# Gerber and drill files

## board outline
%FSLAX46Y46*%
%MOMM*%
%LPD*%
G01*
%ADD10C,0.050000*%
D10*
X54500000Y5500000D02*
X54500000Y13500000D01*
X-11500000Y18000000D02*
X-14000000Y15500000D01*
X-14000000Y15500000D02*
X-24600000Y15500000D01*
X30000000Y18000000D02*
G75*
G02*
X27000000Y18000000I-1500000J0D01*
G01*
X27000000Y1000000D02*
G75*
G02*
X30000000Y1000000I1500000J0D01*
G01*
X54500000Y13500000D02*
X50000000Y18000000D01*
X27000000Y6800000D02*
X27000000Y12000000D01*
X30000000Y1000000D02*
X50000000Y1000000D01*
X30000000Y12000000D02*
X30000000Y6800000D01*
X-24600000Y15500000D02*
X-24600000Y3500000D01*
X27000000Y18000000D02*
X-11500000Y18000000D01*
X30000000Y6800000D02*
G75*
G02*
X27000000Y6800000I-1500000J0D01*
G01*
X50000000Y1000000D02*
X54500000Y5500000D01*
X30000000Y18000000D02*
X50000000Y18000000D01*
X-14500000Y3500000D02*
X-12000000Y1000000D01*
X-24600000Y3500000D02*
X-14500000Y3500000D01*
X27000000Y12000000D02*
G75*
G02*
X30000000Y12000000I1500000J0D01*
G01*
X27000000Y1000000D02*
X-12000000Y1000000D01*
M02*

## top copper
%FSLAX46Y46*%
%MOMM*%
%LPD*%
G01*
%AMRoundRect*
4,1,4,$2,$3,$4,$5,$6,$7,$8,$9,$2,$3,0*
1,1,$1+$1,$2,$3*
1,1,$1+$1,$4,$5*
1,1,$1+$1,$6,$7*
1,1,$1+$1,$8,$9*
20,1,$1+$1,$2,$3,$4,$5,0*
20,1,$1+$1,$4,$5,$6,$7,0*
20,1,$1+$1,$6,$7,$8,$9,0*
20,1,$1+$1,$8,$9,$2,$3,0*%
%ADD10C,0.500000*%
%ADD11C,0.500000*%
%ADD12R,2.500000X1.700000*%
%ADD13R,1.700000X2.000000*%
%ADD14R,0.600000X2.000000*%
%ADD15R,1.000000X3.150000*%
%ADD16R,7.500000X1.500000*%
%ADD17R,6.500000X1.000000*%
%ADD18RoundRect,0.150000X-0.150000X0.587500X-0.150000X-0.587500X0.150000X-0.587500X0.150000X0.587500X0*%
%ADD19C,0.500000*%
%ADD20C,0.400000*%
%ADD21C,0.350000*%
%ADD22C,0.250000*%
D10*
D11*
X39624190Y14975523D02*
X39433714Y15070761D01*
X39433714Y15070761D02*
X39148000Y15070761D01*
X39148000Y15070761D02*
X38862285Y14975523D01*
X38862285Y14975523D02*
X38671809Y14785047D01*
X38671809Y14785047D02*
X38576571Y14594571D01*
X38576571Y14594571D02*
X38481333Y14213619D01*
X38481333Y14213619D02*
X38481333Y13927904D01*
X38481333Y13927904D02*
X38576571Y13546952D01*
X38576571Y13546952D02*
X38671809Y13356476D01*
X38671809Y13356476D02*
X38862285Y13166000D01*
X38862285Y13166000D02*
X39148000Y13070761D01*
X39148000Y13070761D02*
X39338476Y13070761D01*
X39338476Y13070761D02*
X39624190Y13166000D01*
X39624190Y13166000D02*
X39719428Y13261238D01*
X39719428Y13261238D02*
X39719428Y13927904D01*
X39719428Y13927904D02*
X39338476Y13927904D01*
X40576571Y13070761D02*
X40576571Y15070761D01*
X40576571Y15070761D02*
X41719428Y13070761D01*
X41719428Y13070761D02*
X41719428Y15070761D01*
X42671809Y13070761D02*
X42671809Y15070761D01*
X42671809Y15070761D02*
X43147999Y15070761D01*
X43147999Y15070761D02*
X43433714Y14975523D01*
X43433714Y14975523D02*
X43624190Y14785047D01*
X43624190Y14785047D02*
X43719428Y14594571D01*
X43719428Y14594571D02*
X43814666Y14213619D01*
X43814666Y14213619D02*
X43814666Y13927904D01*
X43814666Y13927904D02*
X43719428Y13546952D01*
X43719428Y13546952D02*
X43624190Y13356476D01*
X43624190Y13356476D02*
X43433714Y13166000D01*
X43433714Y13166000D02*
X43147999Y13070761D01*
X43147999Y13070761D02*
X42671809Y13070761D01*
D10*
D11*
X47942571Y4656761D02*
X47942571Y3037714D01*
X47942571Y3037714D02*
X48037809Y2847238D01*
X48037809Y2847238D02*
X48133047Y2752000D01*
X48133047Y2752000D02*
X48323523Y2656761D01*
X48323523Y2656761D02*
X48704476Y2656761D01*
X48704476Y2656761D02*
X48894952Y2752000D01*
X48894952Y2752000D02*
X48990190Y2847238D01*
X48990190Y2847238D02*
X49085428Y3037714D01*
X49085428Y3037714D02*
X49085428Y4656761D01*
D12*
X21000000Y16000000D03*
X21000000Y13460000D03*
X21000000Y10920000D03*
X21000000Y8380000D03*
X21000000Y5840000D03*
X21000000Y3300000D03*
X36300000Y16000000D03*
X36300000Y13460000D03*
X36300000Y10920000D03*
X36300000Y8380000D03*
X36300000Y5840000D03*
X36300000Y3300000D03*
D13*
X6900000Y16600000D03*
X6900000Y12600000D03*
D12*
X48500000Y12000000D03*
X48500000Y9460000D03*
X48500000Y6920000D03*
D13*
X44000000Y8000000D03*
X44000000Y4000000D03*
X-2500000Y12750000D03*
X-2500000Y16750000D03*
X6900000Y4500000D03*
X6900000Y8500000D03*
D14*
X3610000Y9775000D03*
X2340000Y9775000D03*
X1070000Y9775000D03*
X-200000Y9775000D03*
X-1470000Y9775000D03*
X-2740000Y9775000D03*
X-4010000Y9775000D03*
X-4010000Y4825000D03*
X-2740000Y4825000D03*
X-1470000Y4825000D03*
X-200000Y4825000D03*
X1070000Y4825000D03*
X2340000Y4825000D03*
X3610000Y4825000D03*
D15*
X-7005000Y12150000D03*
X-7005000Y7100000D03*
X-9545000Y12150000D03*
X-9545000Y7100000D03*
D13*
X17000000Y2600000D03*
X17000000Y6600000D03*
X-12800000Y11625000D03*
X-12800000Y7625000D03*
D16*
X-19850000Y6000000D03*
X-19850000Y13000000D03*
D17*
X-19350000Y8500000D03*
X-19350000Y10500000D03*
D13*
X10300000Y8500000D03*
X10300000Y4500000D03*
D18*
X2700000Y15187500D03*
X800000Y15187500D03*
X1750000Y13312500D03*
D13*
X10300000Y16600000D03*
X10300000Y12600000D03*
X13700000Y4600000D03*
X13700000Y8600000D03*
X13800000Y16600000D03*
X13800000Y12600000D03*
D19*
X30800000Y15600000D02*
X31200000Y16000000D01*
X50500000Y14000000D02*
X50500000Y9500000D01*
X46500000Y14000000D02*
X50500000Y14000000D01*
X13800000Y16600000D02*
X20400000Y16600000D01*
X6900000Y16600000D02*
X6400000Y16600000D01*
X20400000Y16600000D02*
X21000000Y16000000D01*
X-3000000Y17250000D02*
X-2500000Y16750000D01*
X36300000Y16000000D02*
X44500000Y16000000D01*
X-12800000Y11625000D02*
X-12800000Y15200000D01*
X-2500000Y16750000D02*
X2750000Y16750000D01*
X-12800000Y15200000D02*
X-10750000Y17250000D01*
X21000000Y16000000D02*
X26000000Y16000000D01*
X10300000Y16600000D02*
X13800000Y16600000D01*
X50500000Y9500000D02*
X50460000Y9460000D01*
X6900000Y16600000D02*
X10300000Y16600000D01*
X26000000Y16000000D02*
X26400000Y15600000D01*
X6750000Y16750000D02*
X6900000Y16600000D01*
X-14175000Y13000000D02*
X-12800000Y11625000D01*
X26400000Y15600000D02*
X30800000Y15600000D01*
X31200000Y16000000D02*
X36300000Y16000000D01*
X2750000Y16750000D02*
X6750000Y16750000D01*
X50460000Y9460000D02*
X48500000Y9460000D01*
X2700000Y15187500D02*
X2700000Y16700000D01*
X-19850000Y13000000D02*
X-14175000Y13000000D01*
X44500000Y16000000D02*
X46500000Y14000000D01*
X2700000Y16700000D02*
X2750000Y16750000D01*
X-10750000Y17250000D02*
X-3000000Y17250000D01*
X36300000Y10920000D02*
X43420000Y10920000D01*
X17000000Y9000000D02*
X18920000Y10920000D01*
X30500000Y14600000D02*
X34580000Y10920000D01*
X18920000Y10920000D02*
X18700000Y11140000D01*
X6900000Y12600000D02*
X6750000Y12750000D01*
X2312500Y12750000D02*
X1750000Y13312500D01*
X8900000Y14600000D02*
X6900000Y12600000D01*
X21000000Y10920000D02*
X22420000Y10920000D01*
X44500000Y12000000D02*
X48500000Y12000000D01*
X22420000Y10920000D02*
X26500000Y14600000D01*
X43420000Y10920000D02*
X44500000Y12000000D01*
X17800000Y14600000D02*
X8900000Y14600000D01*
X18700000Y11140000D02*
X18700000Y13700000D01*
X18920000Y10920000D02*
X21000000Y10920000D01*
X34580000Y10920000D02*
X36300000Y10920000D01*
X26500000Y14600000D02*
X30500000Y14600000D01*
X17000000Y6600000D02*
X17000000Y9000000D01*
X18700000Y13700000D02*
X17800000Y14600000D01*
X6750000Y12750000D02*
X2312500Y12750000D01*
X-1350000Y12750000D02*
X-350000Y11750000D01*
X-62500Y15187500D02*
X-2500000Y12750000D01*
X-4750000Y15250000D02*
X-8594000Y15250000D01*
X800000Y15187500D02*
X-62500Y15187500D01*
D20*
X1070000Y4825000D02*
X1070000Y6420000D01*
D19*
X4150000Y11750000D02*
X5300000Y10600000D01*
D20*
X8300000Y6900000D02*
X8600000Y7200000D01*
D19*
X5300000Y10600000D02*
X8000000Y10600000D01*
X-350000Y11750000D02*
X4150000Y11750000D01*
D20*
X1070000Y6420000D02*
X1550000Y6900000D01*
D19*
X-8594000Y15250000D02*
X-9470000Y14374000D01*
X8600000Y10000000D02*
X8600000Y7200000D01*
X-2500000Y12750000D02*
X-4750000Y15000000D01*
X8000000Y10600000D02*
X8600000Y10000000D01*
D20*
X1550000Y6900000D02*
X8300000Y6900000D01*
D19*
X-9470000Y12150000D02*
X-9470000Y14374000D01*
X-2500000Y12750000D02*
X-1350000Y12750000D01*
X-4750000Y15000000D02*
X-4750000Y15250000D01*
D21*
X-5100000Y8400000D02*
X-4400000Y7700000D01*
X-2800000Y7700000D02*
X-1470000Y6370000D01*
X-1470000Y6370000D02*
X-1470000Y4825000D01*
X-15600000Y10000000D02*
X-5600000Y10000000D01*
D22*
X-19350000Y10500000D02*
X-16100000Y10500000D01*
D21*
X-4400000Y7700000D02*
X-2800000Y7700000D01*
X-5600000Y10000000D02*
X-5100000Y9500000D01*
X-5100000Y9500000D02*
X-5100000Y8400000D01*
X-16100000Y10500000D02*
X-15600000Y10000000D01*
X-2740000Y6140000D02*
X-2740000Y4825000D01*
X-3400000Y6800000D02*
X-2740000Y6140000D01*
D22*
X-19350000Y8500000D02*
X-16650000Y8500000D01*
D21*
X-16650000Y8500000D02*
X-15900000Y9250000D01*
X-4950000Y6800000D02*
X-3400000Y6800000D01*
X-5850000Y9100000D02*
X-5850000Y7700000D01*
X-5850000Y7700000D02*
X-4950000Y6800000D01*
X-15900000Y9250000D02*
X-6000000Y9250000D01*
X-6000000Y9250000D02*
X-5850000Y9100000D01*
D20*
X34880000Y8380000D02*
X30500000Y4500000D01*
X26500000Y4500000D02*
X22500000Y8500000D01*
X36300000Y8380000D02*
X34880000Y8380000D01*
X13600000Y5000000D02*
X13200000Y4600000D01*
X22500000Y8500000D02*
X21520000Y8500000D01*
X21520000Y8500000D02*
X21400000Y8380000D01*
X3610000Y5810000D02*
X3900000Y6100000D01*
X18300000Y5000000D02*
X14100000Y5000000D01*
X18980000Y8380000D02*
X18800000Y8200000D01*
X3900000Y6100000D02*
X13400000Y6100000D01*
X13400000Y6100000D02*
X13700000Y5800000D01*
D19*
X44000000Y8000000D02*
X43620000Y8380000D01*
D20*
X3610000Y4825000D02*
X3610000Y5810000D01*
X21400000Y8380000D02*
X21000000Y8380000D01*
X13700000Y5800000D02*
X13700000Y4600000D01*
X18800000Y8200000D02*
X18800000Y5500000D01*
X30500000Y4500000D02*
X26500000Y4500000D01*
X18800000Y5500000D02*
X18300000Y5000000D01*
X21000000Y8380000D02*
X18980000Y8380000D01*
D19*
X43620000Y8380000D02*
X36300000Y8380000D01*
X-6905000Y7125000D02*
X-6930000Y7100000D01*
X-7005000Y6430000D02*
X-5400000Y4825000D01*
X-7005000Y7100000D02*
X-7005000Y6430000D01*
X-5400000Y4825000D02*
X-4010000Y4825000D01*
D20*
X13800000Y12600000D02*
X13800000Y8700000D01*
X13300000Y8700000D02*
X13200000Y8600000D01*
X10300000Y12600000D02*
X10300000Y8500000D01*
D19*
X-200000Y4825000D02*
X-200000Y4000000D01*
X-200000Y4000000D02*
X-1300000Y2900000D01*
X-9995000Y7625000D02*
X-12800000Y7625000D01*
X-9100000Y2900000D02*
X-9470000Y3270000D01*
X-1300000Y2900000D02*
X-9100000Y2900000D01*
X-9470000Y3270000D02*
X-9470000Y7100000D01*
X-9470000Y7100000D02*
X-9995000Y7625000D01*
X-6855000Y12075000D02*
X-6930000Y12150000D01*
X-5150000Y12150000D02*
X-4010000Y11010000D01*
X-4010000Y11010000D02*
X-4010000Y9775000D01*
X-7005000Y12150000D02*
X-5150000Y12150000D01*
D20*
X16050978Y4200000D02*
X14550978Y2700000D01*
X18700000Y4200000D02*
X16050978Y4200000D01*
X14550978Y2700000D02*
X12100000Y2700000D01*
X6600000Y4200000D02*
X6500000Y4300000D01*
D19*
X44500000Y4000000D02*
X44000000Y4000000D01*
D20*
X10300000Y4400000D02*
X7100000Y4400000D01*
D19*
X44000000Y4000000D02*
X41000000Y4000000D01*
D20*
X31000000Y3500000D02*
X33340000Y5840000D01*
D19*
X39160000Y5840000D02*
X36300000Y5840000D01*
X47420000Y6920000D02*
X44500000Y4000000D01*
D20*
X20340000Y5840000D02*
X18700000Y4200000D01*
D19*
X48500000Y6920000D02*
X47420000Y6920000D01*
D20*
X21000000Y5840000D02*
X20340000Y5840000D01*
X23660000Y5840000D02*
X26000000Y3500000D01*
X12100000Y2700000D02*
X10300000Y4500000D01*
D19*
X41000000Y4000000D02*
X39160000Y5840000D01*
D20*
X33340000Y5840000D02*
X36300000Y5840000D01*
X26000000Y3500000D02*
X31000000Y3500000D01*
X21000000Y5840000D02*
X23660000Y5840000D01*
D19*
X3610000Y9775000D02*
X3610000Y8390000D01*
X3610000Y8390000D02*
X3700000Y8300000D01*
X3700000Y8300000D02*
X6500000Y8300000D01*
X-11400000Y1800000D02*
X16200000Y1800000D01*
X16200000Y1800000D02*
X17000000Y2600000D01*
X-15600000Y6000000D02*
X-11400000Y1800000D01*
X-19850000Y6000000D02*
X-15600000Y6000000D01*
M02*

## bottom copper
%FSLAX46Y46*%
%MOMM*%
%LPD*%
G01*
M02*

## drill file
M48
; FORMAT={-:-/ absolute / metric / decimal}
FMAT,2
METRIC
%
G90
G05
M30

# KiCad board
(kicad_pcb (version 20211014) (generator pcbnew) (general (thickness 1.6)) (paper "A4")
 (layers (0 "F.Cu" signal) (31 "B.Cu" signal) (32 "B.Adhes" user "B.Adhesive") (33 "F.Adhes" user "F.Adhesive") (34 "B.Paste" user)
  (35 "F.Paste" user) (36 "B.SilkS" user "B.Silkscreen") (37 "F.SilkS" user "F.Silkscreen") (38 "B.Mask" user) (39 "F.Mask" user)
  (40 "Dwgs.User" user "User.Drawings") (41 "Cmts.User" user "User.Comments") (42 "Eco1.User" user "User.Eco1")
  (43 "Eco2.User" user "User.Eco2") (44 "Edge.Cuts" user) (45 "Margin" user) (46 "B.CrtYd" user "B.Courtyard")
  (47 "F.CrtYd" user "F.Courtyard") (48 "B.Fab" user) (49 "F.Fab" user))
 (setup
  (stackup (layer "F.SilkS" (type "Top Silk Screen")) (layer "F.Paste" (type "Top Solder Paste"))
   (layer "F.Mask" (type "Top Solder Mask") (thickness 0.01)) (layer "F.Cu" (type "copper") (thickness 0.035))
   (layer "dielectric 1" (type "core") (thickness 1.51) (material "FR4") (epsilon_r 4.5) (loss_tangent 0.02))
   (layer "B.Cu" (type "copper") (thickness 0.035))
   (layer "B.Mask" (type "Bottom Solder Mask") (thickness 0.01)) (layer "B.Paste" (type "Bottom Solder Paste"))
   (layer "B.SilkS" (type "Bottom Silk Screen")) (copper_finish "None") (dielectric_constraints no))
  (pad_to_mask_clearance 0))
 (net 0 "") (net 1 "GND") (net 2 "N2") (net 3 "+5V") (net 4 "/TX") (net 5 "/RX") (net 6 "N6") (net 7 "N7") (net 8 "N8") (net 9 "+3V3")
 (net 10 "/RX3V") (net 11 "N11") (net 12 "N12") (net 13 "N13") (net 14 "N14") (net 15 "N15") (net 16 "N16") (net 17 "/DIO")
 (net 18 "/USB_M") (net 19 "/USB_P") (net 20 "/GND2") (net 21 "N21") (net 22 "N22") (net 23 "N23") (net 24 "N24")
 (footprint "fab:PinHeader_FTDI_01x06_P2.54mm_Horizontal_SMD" (layer "F.Cu") (at 21 -16)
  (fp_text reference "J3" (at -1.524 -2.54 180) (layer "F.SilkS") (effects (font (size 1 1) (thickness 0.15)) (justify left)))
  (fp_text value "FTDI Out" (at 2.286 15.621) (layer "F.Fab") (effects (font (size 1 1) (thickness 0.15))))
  (pad "1" smd rect locked (at 0 0) (size 2.5 1.7) (layers "F.Cu" "F.Paste" "F.Mask") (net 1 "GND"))
  (pad "2" smd rect locked (at 0 2.54) (size 2.5 1.7) (layers "F.Cu" "F.Paste" "F.Mask") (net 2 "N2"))
  (pad "3" smd rect locked (at 0 5.08) (size 2.5 1.7) (layers "F.Cu" "F.Paste" "F.Mask") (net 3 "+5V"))
  (pad "4" smd rect locked (at 0 7.62) (size 2.5 1.7) (layers "F.Cu" "F.Paste" "F.Mask") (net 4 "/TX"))
  (pad "5" smd rect locked (at 0 10.16) (size 2.5 1.7) (layers "F.Cu" "F.Paste" "F.Mask") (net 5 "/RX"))
  (pad "6" smd rect locked (at 0 12.7) (size 2.5 1.7) (layers "F.Cu" "F.Paste" "F.Mask") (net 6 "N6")))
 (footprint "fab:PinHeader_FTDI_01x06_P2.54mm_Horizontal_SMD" (layer "F.Cu") (at 36.3 -16)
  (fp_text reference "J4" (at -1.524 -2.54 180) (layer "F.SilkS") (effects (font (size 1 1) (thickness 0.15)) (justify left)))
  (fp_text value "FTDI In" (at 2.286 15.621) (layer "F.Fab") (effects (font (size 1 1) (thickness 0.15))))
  (pad "1" smd rect locked (at 0 0) (size 2.5 1.7) (layers "F.Cu" "F.Paste" "F.Mask") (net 1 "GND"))
  (pad "2" smd rect locked (at 0 2.54) (size 2.5 1.7) (layers "F.Cu" "F.Paste" "F.Mask") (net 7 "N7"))
  (pad "3" smd rect locked (at 0 5.08) (size 2.5 1.7) (layers "F.Cu" "F.Paste" "F.Mask") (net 3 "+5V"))
  (pad "4" smd rect locked (at 0 7.62) (size 2.5 1.7) (layers "F.Cu" "F.Paste" "F.Mask") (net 4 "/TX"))
  (pad "5" smd rect locked (at 0 10.16) (size 2.5 1.7) (layers "F.Cu" "F.Paste" "F.Mask") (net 5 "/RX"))
  (pad "6" smd rect locked (at 0 12.7) (size 2.5 1.7) (layers "F.Cu" "F.Paste" "F.Mask") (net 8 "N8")))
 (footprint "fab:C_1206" (layer "F.Cu") (at 6.9 -14.6 -90)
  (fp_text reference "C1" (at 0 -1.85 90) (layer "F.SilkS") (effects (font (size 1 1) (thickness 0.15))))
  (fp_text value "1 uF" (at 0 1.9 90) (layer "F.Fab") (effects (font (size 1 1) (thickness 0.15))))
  (pad "1" smd rect locked (at -2 0 270) (size 2 1.7) (layers "F.Cu" "F.Paste" "F.Mask") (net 1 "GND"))
  (pad "2" smd rect locked (at 2 0 270) (size 2 1.7) (layers "F.Cu" "F.Paste" "F.Mask") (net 3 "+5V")))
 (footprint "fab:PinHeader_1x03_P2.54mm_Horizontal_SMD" (layer "F.Cu") (at 48.5 -12)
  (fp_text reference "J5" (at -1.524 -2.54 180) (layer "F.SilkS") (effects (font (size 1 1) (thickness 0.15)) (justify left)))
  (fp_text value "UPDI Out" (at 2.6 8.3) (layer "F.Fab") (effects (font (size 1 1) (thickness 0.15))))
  (pad "1" smd rect locked (at 0 0) (size 2.5 1.7) (layers "F.Cu" "F.Paste" "F.Mask") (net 3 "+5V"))
  (pad "2" smd rect locked (at 0 2.54) (size 2.5 1.7) (layers "F.Cu" "F.Paste" "F.Mask") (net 1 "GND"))
  (pad "3" smd rect locked (at 0 5.08) (size 2.5 1.7) (layers "F.Cu" "F.Paste" "F.Mask") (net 5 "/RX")))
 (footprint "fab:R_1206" (layer "F.Cu") (at 44 -6 -90)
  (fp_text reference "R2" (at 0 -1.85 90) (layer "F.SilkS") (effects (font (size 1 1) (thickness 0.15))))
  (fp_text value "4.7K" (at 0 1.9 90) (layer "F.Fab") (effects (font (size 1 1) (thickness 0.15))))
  (pad "1" smd rect locked (at -2 0 270) (size 2 1.7) (layers "F.Cu" "F.Paste" "F.Mask") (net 4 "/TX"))
  (pad "2" smd rect locked (at 2 0 270) (size 2 1.7) (layers "F.Cu" "F.Paste" "F.Mask") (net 5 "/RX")))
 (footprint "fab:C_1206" (layer "F.Cu") (at -2.5 -14.75 90)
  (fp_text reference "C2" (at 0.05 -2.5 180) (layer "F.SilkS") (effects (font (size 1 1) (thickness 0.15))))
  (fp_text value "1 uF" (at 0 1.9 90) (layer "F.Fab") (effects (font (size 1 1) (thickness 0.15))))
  (pad "1" smd rect locked (at -2 0 90) (size 2 1.7) (layers "F.Cu" "F.Paste" "F.Mask") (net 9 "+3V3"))
  (pad "2" smd rect locked (at 2 0 90) (size 2 1.7) (layers "F.Cu" "F.Paste" "F.Mask") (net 1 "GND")))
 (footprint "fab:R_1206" (layer "F.Cu") (at 6.9 -6.5 90)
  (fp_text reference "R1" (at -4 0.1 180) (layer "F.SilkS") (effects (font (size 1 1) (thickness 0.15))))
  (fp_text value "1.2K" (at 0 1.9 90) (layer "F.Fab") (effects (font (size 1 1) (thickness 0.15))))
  (pad "1" smd rect locked (at -2 0 90) (size 2 1.7) (layers "F.Cu" "F.Paste" "F.Mask") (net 5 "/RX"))
  (pad "2" smd rect locked (at 2 0 90) (size 2 1.7) (layers "F.Cu" "F.Paste" "F.Mask") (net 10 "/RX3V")))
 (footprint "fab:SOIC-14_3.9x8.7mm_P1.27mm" (layer "F.Cu") (at -0.2 -7.3 -90)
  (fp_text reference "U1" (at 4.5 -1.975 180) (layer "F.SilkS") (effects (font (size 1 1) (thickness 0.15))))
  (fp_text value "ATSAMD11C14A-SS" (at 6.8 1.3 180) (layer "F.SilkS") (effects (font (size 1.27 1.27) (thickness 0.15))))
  (pad "1" smd rect locked (at -2.475 -3.81 270) (size 2 0.6) (layers "F.Cu" "F.Paste" "F.Mask") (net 10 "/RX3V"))
  (pad "2" smd rect locked (at -2.475 -2.54 270) (size 2 0.6) (layers "F.Cu" "F.Paste" "F.Mask") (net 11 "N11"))
  (pad "3" smd rect locked (at -2.475 -1.27 270) (size 2 0.6) (layers "F.Cu" "F.Paste" "F.Mask") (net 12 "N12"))
  (pad "4" smd rect locked (at -2.475 0 270) (size 2 0.6) (layers "F.Cu" "F.Paste" "F.Mask") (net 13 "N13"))
  (pad "5" smd rect locked (at -2.475 1.27 270) (size 2 0.6) (layers "F.Cu" "F.Paste" "F.Mask") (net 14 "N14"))
  (pad "6" smd rect locked (at -2.475 2.54 270) (size 2 0.6) (layers "F.Cu" "F.Paste" "F.Mask") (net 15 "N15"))
  (pad "7" smd rect locked (at -2.475 3.81 270) (size 2 0.6) (layers "F.Cu" "F.Paste" "F.Mask") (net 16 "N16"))
  (pad "8" smd rect locked (at 2.475 3.81 270) (size 2 0.6) (layers "F.Cu" "F.Paste" "F.Mask") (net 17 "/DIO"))
  (pad "9" smd rect locked (at 2.475 2.54 270) (size 2 0.6) (layers "F.Cu" "F.Paste" "F.Mask") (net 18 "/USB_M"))
  (pad "10" smd rect locked (at 2.475 1.27 270) (size 2 0.6) (layers "F.Cu" "F.Paste" "F.Mask") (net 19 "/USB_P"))
  (pad "11" smd rect locked (at 2.475 0 270) (size 2 0.6) (layers "F.Cu" "F.Paste" "F.Mask") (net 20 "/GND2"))
  (pad "12" smd rect locked (at 2.475 -1.27 270) (size 2 0.6) (layers "F.Cu" "F.Paste" "F.Mask") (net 9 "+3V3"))
  (pad "13" smd rect locked (at 2.475 -2.54 270) (size 2 0.6) (layers "F.Cu" "F.Paste" "F.Mask") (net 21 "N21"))
  (pad "14" smd rect locked (at 2.475 -3.81 270) (size 2 0.6) (layers "F.Cu" "F.Paste" "F.Mask") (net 4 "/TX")))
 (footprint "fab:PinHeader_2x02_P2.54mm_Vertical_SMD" (layer "F.Cu") (at -8.275 -9.625 -90)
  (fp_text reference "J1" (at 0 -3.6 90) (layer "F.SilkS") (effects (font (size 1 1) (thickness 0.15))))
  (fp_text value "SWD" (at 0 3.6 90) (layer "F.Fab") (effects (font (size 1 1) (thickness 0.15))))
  (pad "1" smd rect locked (at -2.525 -1.27 270) (size 3.15 1) (layers "F.Cu" "F.Paste" "F.Mask") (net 16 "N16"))
  (pad "2" smd rect locked (at 2.525 -1.27 270) (size 3.15 1) (layers "F.Cu" "F.Paste" "F.Mask") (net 17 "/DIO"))
  (pad "3" smd rect locked (at -2.525 1.27 270) (size 3.15 1) (layers "F.Cu" "F.Paste" "F.Mask") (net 9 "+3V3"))
  (pad "4" smd rect locked (at 2.525 1.27 270) (size 3.15 1) (layers "F.Cu" "F.Paste" "F.Mask") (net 20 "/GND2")))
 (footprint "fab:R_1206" (layer "F.Cu") (at 17 -4.6 90)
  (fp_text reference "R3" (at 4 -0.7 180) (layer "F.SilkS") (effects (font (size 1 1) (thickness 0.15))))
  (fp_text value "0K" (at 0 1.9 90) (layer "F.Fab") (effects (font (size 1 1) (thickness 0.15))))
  (pad "1" smd rect locked (at -2 0 90) (size 2 1.7) (layers "F.Cu" "F.Paste" "F.Mask") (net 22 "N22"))
  (pad "2" smd rect locked (at 2 0 90) (size 2 1.7) (layers "F.Cu" "F.Paste" "F.Mask") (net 3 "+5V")))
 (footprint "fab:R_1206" (layer "F.Cu") (at -12.8 -9.625 -90)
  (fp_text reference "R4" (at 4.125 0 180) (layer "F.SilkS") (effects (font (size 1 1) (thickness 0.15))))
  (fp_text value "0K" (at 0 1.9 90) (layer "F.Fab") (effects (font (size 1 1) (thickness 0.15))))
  (pad "1" smd rect locked (at -2 0 270) (size 2 1.7) (layers "F.Cu" "F.Paste" "F.Mask") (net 1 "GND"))
  (pad "2" smd rect locked (at 2 0 270) (size 2 1.7) (layers "F.Cu" "F.Paste" "F.Mask") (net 20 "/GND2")))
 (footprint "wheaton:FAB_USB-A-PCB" (layer "F.Cu") (at -19.65 -9.5)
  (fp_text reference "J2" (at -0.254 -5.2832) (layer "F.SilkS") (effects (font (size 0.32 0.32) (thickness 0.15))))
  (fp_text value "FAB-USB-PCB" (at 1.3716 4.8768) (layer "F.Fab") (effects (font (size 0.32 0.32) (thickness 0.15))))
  (pad "5V" smd rect locked (at -0.2 3.5) (size 7.5 1.5) (layers "F.Cu" "F.Paste" "F.Mask") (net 22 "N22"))
  (pad "GND" smd rect locked (at -0.2 -3.5) (size 7.5 1.5) (layers "F.Cu" "F.Paste" "F.Mask") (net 1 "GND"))
  (pad "USB_M" smd rect locked (at 0.3 1) (size 6.5 1) (layers "F.Cu" "F.Paste" "F.Mask") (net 18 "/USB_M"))
  (pad "USB_P" smd rect locked (at 0.3 -1) (size 6.5 1) (layers "F.Cu" "F.Paste" "F.Mask") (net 19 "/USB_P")))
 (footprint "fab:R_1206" (layer "F.Cu") (at 10.3 -6.5 -90)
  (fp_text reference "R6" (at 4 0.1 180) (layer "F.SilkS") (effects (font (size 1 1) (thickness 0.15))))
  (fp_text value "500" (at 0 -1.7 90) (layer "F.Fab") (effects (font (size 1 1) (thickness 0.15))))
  (pad "1" smd rect locked (at -2 0 270) (size 2 1.7) (layers "F.Cu" "F.Paste" "F.Mask") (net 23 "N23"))
  (pad "2" smd rect locked (at 2 0 270) (size 2 1.7) (layers "F.Cu" "F.Paste" "F.Mask") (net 5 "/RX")))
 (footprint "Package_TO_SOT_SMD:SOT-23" (layer "F.Cu") (at 1.75 -14.25 -90)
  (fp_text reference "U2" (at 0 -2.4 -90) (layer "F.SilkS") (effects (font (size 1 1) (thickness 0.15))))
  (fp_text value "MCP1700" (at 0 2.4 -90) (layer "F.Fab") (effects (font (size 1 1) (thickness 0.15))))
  (pad "1" smd roundrect (at -0.9375 -0.95 270) (size 1.475 0.6) (layers "F.Cu" "F.Paste" "F.Mask") (roundrect_rratio 0.25) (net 1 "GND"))
  (pad "2" smd roundrect (at -0.9375 0.95 270) (size 1.475 0.6) (layers "F.Cu" "F.Paste" "F.Mask") (roundrect_rratio 0.25) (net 9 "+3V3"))
  (pad "3" smd roundrect (at 0.9375 0 270) (size 1.475 0.6) (layers "F.Cu" "F.Paste" "F.Mask") (roundrect_rratio 0.25) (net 3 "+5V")))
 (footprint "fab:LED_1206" (layer "F.Cu") (at 10.3 -14.6 -90)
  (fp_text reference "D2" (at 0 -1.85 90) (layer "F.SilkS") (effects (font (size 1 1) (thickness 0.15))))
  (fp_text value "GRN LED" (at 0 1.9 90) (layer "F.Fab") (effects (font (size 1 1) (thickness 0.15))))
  (pad "1" smd rect locked (at -2 0 270) (size 2 1.7) (layers "F.Cu" "F.Paste" "F.Mask") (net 1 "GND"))
  (pad "2" smd rect locked (at 2 0 270) (size 2 1.7) (layers "F.Cu" "F.Paste" "F.Mask") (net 23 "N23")))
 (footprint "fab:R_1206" (layer "F.Cu") (at 13.7 -6.6 90)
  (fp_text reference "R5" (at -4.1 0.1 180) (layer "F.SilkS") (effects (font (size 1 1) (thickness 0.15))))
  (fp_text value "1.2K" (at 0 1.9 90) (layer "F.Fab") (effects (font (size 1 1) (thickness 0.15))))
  (pad "1" smd rect locked (at -2 0 90) (size 2 1.7) (layers "F.Cu" "F.Paste" "F.Mask") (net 4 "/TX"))
  (pad "2" smd rect locked (at 2 0 90) (size 2 1.7) (layers "F.Cu" "F.Paste" "F.Mask") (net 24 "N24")))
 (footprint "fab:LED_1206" (layer "F.Cu") (at 13.8 -14.6 -90)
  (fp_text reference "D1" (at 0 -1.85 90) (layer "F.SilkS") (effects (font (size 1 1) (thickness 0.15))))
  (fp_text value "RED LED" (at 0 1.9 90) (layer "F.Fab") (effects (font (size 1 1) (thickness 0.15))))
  (pad "1" smd rect locked (at -2 0 270) (size 2 1.7) (layers "F.Cu" "F.Paste" "F.Mask") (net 1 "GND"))
  (pad "2" smd rect locked (at 2 0 270) (size 2 1.7) (layers "F.Cu" "F.Paste" "F.Mask") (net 24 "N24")))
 (gr_line (start 54.5 -5.5) (end 54.5 -13.5) (layer "Edge.Cuts") (width 0.05))
 (gr_line (start -11.5 -18) (end -14 -15.5) (layer "Edge.Cuts") (width 0.05))
 (gr_line (start -14 -15.5) (end -24.6 -15.5) (layer "Edge.Cuts") (width 0.05))
 (gr_arc (start 30 -18) (mid 28.5 -16.5) (end 27 -18) (layer "Edge.Cuts") (width 0.05))
 (gr_arc (start 27 -1) (mid 28.5 -2.5) (end 30 -1) (layer "Edge.Cuts") (width 0.05))
 (gr_line (start 54.5 -13.5) (end 50 -18) (layer "Edge.Cuts") (width 0.05))
 (gr_line (start 27 -6.8) (end 27 -12) (layer "Edge.Cuts") (width 0.05))
 (gr_line (start 30 -1) (end 50 -1) (layer "Edge.Cuts") (width 0.05))
 (gr_line (start 30 -12) (end 30 -6.8) (layer "Edge.Cuts") (width 0.05))
 (gr_line (start -24.6 -15.5) (end -24.6 -3.5) (layer "Edge.Cuts") (width 0.05))
 (gr_line (start 27 -18) (end -11.5 -18) (layer "Edge.Cuts") (width 0.05))
 (gr_arc (start 30 -6.8) (mid 28.5 -5.3) (end 27 -6.8) (layer "Edge.Cuts") (width 0.05))
 (gr_line (start 50 -1) (end 54.5 -5.5) (layer "Edge.Cuts") (width 0.05))
 (gr_line (start 30 -18) (end 50 -18) (layer "Edge.Cuts") (width 0.05))
 (gr_line (start -14.5 -3.5) (end -12 -1) (layer "Edge.Cuts") (width 0.05))
 (gr_line (start -24.6 -3.5) (end -14.5 -3.5) (layer "Edge.Cuts") (width 0.05))
 (gr_arc (start 27 -12) (mid 28.5 -13.5) (end 30 -12) (layer "Edge.Cuts") (width 0.05))
 (gr_line (start 27 -1) (end -12 -1) (layer "Edge.Cuts") (width 0.05))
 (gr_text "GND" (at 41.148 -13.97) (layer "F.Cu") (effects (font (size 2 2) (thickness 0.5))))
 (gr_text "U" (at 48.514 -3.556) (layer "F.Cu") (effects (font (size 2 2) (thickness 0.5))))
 (segment (start 30.8 -15.6) (end 31.2 -16) (width 0.5) (layer "F.Cu") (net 1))
 (segment (start 50.5 -14) (end 50.5 -9.5) (width 0.5) (layer "F.Cu") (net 1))
 (segment (start 46.5 -14) (end 50.5 -14) (width 0.5) (layer "F.Cu") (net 1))
 (segment (start 13.8 -16.6) (end 20.4 -16.6) (width 0.5) (layer "F.Cu") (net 1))
 (segment (start 6.9 -16.6) (end 6.4 -16.6) (width 0.5) (layer "F.Cu") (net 1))
 (segment (start 20.4 -16.6) (end 21 -16) (width 0.5) (layer "F.Cu") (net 1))
 (segment (start -3 -17.25) (end -2.5 -16.75) (width 0.5) (layer "F.Cu") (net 1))
 (segment (start 36.3 -16) (end 44.5 -16) (width 0.5) (layer "F.Cu") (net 1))
 (segment (start -12.8 -11.625) (end -12.8 -15.2) (width 0.5) (layer "F.Cu") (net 1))
 (segment (start -2.5 -16.75) (end 2.75 -16.75) (width 0.5) (layer "F.Cu") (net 1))
 (segment (start -12.8 -15.2) (end -10.75 -17.25) (width 0.5) (layer "F.Cu") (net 1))
 (segment (start 21 -16) (end 26 -16) (width 0.5) (layer "F.Cu") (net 1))
 (segment (start 10.3 -16.6) (end 13.8 -16.6) (width 0.5) (layer "F.Cu") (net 1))
 (segment (start 50.5 -9.5) (end 50.46 -9.46) (width 0.5) (layer "F.Cu") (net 1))
 (segment (start 6.9 -16.6) (end 10.3 -16.6) (width 0.5) (layer "F.Cu") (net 1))
 (segment (start 26 -16) (end 26.4 -15.6) (width 0.5) (layer "F.Cu") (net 1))
 (segment (start 6.75 -16.75) (end 6.9 -16.6) (width 0.5) (layer "F.Cu") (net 1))
 (segment (start -14.175 -13) (end -12.8 -11.625) (width 0.5) (layer "F.Cu") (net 1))
 (segment (start 26.4 -15.6) (end 30.8 -15.6) (width 0.5) (layer "F.Cu") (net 1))
 (segment (start 31.2 -16) (end 36.3 -16) (width 0.5) (layer "F.Cu") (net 1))
 (segment (start 2.75 -16.75) (end 6.75 -16.75) (width 0.5) (layer "F.Cu") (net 1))
 (segment (start 50.46 -9.46) (end 48.5 -9.46) (width 0.5) (layer "F.Cu") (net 1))
 (segment (start 2.7 -15.1875) (end 2.7 -16.7) (width 0.5) (layer "F.Cu") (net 1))
 (segment (start -19.85 -13) (end -14.175 -13) (width 0.5) (layer "F.Cu") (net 1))
 (segment (start 44.5 -16) (end 46.5 -14) (width 0.5) (layer "F.Cu") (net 1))
 (segment (start 2.7 -16.7) (end 2.75 -16.75) (width 0.5) (layer "F.Cu") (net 1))
 (segment (start -10.75 -17.25) (end -3 -17.25) (width 0.5) (layer "F.Cu") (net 1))
 (segment (start 36.3 -10.92) (end 43.42 -10.92) (width 0.5) (layer "F.Cu") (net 3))
 (segment (start 17 -9) (end 18.92 -10.92) (width 0.5) (layer "F.Cu") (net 3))
 (segment (start 30.5 -14.6) (end 34.58 -10.92) (width 0.5) (layer "F.Cu") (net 3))
 (segment (start 18.92 -10.92) (end 18.7 -11.14) (width 0.5) (layer "F.Cu") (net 3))
 (segment (start 6.9 -12.6) (end 6.75 -12.75) (width 0.5) (layer "F.Cu") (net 3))
 (segment (start 2.3125 -12.75) (end 1.75 -13.3125) (width 0.5) (layer "F.Cu") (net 3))
 (segment (start 8.9 -14.6) (end 6.9 -12.6) (width 0.5) (layer "F.Cu") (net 3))
 (segment (start 21 -10.92) (end 22.42 -10.92) (width 0.5) (layer "F.Cu") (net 3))
 (segment (start 44.5 -12) (end 48.5 -12) (width 0.5) (layer "F.Cu") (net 3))
 (segment (start 22.42 -10.92) (end 26.5 -14.6) (width 0.5) (layer "F.Cu") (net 3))
 (segment (start 43.42 -10.92) (end 44.5 -12) (width 0.5) (layer "F.Cu") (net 3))
 (segment (start 17.8 -14.6) (end 8.9 -14.6) (width 0.5) (layer "F.Cu") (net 3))
 (segment (start 18.7 -11.14) (end 18.7 -13.7) (width 0.5) (layer "F.Cu") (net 3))
 (segment (start 18.92 -10.92) (end 21 -10.92) (width 0.5) (layer "F.Cu") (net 3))
 (segment (start 34.58 -10.92) (end 36.3 -10.92) (width 0.5) (layer "F.Cu") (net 3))
 (segment (start 26.5 -14.6) (end 30.5 -14.6) (width 0.5) (layer "F.Cu") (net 3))
 (segment (start 17 -6.6) (end 17 -9) (width 0.5) (layer "F.Cu") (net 3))
 (segment (start 18.7 -13.7) (end 17.8 -14.6) (width 0.5) (layer "F.Cu") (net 3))
 (segment (start 6.75 -12.75) (end 2.3125 -12.75) (width 0.5) (layer "F.Cu") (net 3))
 (segment (start -1.35 -12.75) (end -0.35 -11.75) (width 0.5) (layer "F.Cu") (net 9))
 (segment (start -0.0625 -15.1875) (end -2.5 -12.75) (width 0.5) (layer "F.Cu") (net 9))
 (segment (start -4.75 -15.25) (end -8.594 -15.25) (width 0.5) (layer "F.Cu") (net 9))
 (segment (start 0.8 -15.1875) (end -0.0625 -15.1875) (width 0.5) (layer "F.Cu") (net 9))
 (segment (start 1.07 -4.825) (end 1.07 -6.42) (width 0.4) (layer "F.Cu") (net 9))
 (segment (start 4.15 -11.75) (end 5.3 -10.6) (width 0.5) (layer "F.Cu") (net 9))
 (segment (start 8.3 -6.9) (end 8.6 -7.2) (width 0.4) (layer "F.Cu") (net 9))
 (segment (start 5.3 -10.6) (end 8 -10.6) (width 0.5) (layer "F.Cu") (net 9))
 (segment (start -0.35 -11.75) (end 4.15 -11.75) (width 0.5) (layer "F.Cu") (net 9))
 (segment (start 1.07 -6.42) (end 1.55 -6.9) (width 0.4) (layer "F.Cu") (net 9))
 (segment (start -8.594 -15.25) (end -9.47 -14.374) (width 0.5) (layer "F.Cu") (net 9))
 (segment (start 8.6 -10) (end 8.6 -7.2) (width 0.5) (layer "F.Cu") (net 9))
 (segment (start -2.5 -12.75) (end -4.75 -15) (width 0.5) (layer "F.Cu") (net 9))
 (segment (start 8 -10.6) (end 8.6 -10) (width 0.5) (layer "F.Cu") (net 9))
 (segment (start 1.55 -6.9) (end 8.3 -6.9) (width 0.4) (layer "F.Cu") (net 9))
 (segment (start -9.47 -12.15) (end -9.47 -14.374) (width 0.5) (layer "F.Cu") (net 9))
 (segment (start -2.5 -12.75) (end -1.35 -12.75) (width 0.5) (layer "F.Cu") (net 9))
 (segment (start -4.75 -15) (end -4.75 -15.25) (width 0.5) (layer "F.Cu") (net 9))
 (segment (start -5.1 -8.4) (end -4.4 -7.7) (width 0.35) (layer "F.Cu") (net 19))
 (segment (start -2.8 -7.7) (end -1.47 -6.37) (width 0.35) (layer "F.Cu") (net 19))
 (segment (start -1.47 -6.37) (end -1.47 -4.825) (width 0.35) (layer "F.Cu") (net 19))
 (segment (start -15.6 -10) (end -5.6 -10) (width 0.35) (layer "F.Cu") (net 19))
 (segment (start -19.35 -10.5) (end -16.1 -10.5) (width 0.25) (layer "F.Cu") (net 19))
 (segment (start -4.4 -7.7) (end -2.8 -7.7) (width 0.35) (layer "F.Cu") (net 19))
 (segment (start -5.6 -10) (end -5.1 -9.5) (width 0.35) (layer "F.Cu") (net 19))
 (segment (start -5.1 -9.5) (end -5.1 -8.4) (width 0.35) (layer "F.Cu") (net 19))
 (segment (start -16.1 -10.5) (end -15.6 -10) (width 0.35) (layer "F.Cu") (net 19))
 (segment (start -2.74 -6.14) (end -2.74 -4.825) (width 0.35) (layer "F.Cu") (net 18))
 (segment (start -3.4 -6.8) (end -2.74 -6.14) (width 0.35) (layer "F.Cu") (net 18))
 (segment (start -19.35 -8.5) (end -16.65 -8.5) (width 0.25) (layer "F.Cu") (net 18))
 (segment (start -16.65 -8.5) (end -15.9 -9.25) (width 0.35) (layer "F.Cu") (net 18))
 (segment (start -4.95 -6.8) (end -3.4 -6.8) (width 0.35) (layer "F.Cu") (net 18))
 (segment (start -5.85 -9.1) (end -5.85 -7.7) (width 0.35) (layer "F.Cu") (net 18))
 (segment (start -5.85 -7.7) (end -4.95 -6.8) (width 0.35) (layer "F.Cu") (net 18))
 (segment (start -15.9 -9.25) (end -6 -9.25) (width 0.35) (layer "F.Cu") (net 18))
 (segment (start -6 -9.25) (end -5.85 -9.1) (width 0.35) (layer "F.Cu") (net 18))
 (segment (start 34.88 -8.38) (end 30.5 -4.5) (width 0.4) (layer "F.Cu") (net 4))
 (segment (start 26.5 -4.5) (end 22.5 -8.5) (width 0.4) (layer "F.Cu") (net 4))
 (segment (start 36.3 -8.38) (end 34.88 -8.38) (width 0.4) (layer "F.Cu") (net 4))
 (segment (start 13.6 -5) (end 13.2 -4.6) (width 0.4) (layer "F.Cu") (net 4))
 (segment (start 22.5 -8.5) (end 21.52 -8.5) (width 0.4) (layer "F.Cu") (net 4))
 (segment (start 21.52 -8.5) (end 21.4 -8.38) (width 0.4) (layer "F.Cu") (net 4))
 (segment (start 3.61 -5.81) (end 3.9 -6.1) (width 0.4) (layer "F.Cu") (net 4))
 (segment (start 18.3 -5) (end 14.1 -5) (width 0.4) (layer "F.Cu") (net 4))
 (segment (start 18.98 -8.38) (end 18.8 -8.2) (width 0.4) (layer "F.Cu") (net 4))
 (segment (start 3.9 -6.1) (end 13.4 -6.1) (width 0.4) (layer "F.Cu") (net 4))
 (segment (start 13.4 -6.1) (end 13.7 -5.8) (width 0.4) (layer "F.Cu") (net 4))
 (segment (start 44 -8) (end 43.62 -8.38) (width 0.5) (layer "F.Cu") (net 4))
 (segment (start 3.61 -4.825) (end 3.61 -5.81) (width 0.4) (layer "F.Cu") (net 4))
 (segment (start 21.4 -8.38) (end 21 -8.38) (width 0.4) (layer "F.Cu") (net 4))
 (segment (start 13.7 -5.8) (end 13.7 -4.6) (width 0.4) (layer "F.Cu") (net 4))
 (segment (start 18.8 -8.2) (end 18.8 -5.5) (width 0.4) (layer "F.Cu") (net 4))
 (segment (start 30.5 -4.5) (end 26.5 -4.5) (width 0.4) (layer "F.Cu") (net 4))
 (segment (start 18.8 -5.5) (end 18.3 -5) (width 0.4) (layer "F.Cu") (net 4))
 (segment (start 21 -8.38) (end 18.98 -8.38) (width 0.4) (layer "F.Cu") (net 4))
 (segment (start 43.62 -8.38) (end 36.3 -8.38) (width 0.5) (layer "F.Cu") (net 4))
 (segment (start -6.905 -7.125) (end -6.93 -7.1) (width 0.5) (layer "F.Cu") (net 17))
 (segment (start -7.005 -6.43) (end -5.4 -4.825) (width 0.5) (layer "F.Cu") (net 17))
 (segment (start -7.005 -7.1) (end -7.005 -6.43) (width 0.5) (layer "F.Cu") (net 17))
 (segment (start -5.4 -4.825) (end -4.01 -4.825) (width 0.5) (layer "F.Cu") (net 17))
 (segment (start 13.8 -12.6) (end 13.8 -8.7) (width 0.4) (layer "F.Cu") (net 24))
 (segment (start 13.3 -8.7) (end 13.2 -8.6) (width 0.4) (layer "F.Cu") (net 24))
 (segment (start 10.3 -12.6) (end 10.3 -8.5) (width 0.4) (layer "F.Cu") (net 23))
 (segment (start -0.2 -4.825) (end -0.2 -4) (width 0.5) (layer "F.Cu") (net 20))
 (segment (start -0.2 -4) (end -1.3 -2.9) (width 0.5) (layer "F.Cu") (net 20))
 (segment (start -9.995 -7.625) (end -12.8 -7.625) (width 0.5) (layer "F.Cu") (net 20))
 (segment (start -9.1 -2.9) (end -9.47 -3.27) (width 0.5) (layer "F.Cu") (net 20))
 (segment (start -1.3 -2.9) (end -9.1 -2.9) (width 0.5) (layer "F.Cu") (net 20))
 (segment (start -9.47 -3.27) (end -9.47 -7.1) (width 0.5) (layer "F.Cu") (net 20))
 (segment (start -9.47 -7.1) (end -9.995 -7.625) (width 0.5) (layer "F.Cu") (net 20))
 (segment (start -6.855 -12.075) (end -6.93 -12.15) (width 0.5) (layer "F.Cu") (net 16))
 (segment (start -5.15 -12.15) (end -4.01 -11.01) (width 0.5) (layer "F.Cu") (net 16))
 (segment (start -4.01 -11.01) (end -4.01 -9.775) (width 0.5) (layer "F.Cu") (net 16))
 (segment (start -7.005 -12.15) (end -5.15 -12.15) (width 0.5) (layer "F.Cu") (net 16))
 (segment (start 16.050978 -4.2) (end 14.550978 -2.7) (width 0.4) (layer "F.Cu") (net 5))
 (segment (start 18.7 -4.2) (end 16.050978 -4.2) (width 0.4) (layer "F.Cu") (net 5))
 (segment (start 14.550978 -2.7) (end 12.1 -2.7) (width 0.4) (layer "F.Cu") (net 5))
 (segment (start 6.6 -4.2) (end 6.5 -4.3) (width 0.4) (layer "F.Cu") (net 5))
 (segment (start 44.5 -4) (end 44 -4) (width 0.5) (layer "F.Cu") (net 5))
 (segment (start 10.3 -4.4) (end 7.1 -4.4) (width 0.4) (layer "F.Cu") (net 5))
 (segment (start 44 -4) (end 41 -4) (width 0.5) (layer "F.Cu") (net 5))
 (segment (start 31 -3.5) (end 33.34 -5.84) (width 0.4) (layer "F.Cu") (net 5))
 (segment (start 39.16 -5.84) (end 36.3 -5.84) (width 0.5) (layer "F.Cu") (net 5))
 (segment (start 47.42 -6.92) (end 44.5 -4) (width 0.5) (layer "F.Cu") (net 5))
 (segment (start 20.34 -5.84) (end 18.7 -4.2) (width 0.4) (layer "F.Cu") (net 5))
 (segment (start 48.5 -6.92) (end 47.42 -6.92) (width 0.5) (layer "F.Cu") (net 5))
 (segment (start 21 -5.84) (end 20.34 -5.84) (width 0.4) (layer "F.Cu") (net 5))
 (segment (start 23.66 -5.84) (end 26 -3.5) (width 0.4) (layer "F.Cu") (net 5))
 (segment (start 12.1 -2.7) (end 10.3 -4.5) (width 0.4) (layer "F.Cu") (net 5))
 (segment (start 41 -4) (end 39.16 -5.84) (width 0.5) (layer "F.Cu") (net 5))
 (segment (start 33.34 -5.84) (end 36.3 -5.84) (width 0.4) (layer "F.Cu") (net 5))
 (segment (start 26 -3.5) (end 31 -3.5) (width 0.4) (layer "F.Cu") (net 5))
 (segment (start 21 -5.84) (end 23.66 -5.84) (width 0.4) (layer "F.Cu") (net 5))
 (segment (start 3.61 -9.775) (end 3.61 -8.39) (width 0.5) (layer "F.Cu") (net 10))
 (segment (start 3.61 -8.39) (end 3.7 -8.3) (width 0.5) (layer "F.Cu") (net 10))
 (segment (start 3.7 -8.3) (end 6.5 -8.3) (width 0.5) (layer "F.Cu") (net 10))
 (segment (start -11.4 -1.8) (end 16.2 -1.8) (width 0.5) (layer "F.Cu") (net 22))
 (segment (start 16.2 -1.8) (end 17 -2.6) (width 0.5) (layer "F.Cu") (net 22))
 (segment (start -15.6 -6) (end -11.4 -1.8) (width 0.5) (layer "F.Cu") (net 22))
 (segment (start -19.85 -6) (end -15.6 -6) (width 0.5) (layer "F.Cu") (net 22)))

